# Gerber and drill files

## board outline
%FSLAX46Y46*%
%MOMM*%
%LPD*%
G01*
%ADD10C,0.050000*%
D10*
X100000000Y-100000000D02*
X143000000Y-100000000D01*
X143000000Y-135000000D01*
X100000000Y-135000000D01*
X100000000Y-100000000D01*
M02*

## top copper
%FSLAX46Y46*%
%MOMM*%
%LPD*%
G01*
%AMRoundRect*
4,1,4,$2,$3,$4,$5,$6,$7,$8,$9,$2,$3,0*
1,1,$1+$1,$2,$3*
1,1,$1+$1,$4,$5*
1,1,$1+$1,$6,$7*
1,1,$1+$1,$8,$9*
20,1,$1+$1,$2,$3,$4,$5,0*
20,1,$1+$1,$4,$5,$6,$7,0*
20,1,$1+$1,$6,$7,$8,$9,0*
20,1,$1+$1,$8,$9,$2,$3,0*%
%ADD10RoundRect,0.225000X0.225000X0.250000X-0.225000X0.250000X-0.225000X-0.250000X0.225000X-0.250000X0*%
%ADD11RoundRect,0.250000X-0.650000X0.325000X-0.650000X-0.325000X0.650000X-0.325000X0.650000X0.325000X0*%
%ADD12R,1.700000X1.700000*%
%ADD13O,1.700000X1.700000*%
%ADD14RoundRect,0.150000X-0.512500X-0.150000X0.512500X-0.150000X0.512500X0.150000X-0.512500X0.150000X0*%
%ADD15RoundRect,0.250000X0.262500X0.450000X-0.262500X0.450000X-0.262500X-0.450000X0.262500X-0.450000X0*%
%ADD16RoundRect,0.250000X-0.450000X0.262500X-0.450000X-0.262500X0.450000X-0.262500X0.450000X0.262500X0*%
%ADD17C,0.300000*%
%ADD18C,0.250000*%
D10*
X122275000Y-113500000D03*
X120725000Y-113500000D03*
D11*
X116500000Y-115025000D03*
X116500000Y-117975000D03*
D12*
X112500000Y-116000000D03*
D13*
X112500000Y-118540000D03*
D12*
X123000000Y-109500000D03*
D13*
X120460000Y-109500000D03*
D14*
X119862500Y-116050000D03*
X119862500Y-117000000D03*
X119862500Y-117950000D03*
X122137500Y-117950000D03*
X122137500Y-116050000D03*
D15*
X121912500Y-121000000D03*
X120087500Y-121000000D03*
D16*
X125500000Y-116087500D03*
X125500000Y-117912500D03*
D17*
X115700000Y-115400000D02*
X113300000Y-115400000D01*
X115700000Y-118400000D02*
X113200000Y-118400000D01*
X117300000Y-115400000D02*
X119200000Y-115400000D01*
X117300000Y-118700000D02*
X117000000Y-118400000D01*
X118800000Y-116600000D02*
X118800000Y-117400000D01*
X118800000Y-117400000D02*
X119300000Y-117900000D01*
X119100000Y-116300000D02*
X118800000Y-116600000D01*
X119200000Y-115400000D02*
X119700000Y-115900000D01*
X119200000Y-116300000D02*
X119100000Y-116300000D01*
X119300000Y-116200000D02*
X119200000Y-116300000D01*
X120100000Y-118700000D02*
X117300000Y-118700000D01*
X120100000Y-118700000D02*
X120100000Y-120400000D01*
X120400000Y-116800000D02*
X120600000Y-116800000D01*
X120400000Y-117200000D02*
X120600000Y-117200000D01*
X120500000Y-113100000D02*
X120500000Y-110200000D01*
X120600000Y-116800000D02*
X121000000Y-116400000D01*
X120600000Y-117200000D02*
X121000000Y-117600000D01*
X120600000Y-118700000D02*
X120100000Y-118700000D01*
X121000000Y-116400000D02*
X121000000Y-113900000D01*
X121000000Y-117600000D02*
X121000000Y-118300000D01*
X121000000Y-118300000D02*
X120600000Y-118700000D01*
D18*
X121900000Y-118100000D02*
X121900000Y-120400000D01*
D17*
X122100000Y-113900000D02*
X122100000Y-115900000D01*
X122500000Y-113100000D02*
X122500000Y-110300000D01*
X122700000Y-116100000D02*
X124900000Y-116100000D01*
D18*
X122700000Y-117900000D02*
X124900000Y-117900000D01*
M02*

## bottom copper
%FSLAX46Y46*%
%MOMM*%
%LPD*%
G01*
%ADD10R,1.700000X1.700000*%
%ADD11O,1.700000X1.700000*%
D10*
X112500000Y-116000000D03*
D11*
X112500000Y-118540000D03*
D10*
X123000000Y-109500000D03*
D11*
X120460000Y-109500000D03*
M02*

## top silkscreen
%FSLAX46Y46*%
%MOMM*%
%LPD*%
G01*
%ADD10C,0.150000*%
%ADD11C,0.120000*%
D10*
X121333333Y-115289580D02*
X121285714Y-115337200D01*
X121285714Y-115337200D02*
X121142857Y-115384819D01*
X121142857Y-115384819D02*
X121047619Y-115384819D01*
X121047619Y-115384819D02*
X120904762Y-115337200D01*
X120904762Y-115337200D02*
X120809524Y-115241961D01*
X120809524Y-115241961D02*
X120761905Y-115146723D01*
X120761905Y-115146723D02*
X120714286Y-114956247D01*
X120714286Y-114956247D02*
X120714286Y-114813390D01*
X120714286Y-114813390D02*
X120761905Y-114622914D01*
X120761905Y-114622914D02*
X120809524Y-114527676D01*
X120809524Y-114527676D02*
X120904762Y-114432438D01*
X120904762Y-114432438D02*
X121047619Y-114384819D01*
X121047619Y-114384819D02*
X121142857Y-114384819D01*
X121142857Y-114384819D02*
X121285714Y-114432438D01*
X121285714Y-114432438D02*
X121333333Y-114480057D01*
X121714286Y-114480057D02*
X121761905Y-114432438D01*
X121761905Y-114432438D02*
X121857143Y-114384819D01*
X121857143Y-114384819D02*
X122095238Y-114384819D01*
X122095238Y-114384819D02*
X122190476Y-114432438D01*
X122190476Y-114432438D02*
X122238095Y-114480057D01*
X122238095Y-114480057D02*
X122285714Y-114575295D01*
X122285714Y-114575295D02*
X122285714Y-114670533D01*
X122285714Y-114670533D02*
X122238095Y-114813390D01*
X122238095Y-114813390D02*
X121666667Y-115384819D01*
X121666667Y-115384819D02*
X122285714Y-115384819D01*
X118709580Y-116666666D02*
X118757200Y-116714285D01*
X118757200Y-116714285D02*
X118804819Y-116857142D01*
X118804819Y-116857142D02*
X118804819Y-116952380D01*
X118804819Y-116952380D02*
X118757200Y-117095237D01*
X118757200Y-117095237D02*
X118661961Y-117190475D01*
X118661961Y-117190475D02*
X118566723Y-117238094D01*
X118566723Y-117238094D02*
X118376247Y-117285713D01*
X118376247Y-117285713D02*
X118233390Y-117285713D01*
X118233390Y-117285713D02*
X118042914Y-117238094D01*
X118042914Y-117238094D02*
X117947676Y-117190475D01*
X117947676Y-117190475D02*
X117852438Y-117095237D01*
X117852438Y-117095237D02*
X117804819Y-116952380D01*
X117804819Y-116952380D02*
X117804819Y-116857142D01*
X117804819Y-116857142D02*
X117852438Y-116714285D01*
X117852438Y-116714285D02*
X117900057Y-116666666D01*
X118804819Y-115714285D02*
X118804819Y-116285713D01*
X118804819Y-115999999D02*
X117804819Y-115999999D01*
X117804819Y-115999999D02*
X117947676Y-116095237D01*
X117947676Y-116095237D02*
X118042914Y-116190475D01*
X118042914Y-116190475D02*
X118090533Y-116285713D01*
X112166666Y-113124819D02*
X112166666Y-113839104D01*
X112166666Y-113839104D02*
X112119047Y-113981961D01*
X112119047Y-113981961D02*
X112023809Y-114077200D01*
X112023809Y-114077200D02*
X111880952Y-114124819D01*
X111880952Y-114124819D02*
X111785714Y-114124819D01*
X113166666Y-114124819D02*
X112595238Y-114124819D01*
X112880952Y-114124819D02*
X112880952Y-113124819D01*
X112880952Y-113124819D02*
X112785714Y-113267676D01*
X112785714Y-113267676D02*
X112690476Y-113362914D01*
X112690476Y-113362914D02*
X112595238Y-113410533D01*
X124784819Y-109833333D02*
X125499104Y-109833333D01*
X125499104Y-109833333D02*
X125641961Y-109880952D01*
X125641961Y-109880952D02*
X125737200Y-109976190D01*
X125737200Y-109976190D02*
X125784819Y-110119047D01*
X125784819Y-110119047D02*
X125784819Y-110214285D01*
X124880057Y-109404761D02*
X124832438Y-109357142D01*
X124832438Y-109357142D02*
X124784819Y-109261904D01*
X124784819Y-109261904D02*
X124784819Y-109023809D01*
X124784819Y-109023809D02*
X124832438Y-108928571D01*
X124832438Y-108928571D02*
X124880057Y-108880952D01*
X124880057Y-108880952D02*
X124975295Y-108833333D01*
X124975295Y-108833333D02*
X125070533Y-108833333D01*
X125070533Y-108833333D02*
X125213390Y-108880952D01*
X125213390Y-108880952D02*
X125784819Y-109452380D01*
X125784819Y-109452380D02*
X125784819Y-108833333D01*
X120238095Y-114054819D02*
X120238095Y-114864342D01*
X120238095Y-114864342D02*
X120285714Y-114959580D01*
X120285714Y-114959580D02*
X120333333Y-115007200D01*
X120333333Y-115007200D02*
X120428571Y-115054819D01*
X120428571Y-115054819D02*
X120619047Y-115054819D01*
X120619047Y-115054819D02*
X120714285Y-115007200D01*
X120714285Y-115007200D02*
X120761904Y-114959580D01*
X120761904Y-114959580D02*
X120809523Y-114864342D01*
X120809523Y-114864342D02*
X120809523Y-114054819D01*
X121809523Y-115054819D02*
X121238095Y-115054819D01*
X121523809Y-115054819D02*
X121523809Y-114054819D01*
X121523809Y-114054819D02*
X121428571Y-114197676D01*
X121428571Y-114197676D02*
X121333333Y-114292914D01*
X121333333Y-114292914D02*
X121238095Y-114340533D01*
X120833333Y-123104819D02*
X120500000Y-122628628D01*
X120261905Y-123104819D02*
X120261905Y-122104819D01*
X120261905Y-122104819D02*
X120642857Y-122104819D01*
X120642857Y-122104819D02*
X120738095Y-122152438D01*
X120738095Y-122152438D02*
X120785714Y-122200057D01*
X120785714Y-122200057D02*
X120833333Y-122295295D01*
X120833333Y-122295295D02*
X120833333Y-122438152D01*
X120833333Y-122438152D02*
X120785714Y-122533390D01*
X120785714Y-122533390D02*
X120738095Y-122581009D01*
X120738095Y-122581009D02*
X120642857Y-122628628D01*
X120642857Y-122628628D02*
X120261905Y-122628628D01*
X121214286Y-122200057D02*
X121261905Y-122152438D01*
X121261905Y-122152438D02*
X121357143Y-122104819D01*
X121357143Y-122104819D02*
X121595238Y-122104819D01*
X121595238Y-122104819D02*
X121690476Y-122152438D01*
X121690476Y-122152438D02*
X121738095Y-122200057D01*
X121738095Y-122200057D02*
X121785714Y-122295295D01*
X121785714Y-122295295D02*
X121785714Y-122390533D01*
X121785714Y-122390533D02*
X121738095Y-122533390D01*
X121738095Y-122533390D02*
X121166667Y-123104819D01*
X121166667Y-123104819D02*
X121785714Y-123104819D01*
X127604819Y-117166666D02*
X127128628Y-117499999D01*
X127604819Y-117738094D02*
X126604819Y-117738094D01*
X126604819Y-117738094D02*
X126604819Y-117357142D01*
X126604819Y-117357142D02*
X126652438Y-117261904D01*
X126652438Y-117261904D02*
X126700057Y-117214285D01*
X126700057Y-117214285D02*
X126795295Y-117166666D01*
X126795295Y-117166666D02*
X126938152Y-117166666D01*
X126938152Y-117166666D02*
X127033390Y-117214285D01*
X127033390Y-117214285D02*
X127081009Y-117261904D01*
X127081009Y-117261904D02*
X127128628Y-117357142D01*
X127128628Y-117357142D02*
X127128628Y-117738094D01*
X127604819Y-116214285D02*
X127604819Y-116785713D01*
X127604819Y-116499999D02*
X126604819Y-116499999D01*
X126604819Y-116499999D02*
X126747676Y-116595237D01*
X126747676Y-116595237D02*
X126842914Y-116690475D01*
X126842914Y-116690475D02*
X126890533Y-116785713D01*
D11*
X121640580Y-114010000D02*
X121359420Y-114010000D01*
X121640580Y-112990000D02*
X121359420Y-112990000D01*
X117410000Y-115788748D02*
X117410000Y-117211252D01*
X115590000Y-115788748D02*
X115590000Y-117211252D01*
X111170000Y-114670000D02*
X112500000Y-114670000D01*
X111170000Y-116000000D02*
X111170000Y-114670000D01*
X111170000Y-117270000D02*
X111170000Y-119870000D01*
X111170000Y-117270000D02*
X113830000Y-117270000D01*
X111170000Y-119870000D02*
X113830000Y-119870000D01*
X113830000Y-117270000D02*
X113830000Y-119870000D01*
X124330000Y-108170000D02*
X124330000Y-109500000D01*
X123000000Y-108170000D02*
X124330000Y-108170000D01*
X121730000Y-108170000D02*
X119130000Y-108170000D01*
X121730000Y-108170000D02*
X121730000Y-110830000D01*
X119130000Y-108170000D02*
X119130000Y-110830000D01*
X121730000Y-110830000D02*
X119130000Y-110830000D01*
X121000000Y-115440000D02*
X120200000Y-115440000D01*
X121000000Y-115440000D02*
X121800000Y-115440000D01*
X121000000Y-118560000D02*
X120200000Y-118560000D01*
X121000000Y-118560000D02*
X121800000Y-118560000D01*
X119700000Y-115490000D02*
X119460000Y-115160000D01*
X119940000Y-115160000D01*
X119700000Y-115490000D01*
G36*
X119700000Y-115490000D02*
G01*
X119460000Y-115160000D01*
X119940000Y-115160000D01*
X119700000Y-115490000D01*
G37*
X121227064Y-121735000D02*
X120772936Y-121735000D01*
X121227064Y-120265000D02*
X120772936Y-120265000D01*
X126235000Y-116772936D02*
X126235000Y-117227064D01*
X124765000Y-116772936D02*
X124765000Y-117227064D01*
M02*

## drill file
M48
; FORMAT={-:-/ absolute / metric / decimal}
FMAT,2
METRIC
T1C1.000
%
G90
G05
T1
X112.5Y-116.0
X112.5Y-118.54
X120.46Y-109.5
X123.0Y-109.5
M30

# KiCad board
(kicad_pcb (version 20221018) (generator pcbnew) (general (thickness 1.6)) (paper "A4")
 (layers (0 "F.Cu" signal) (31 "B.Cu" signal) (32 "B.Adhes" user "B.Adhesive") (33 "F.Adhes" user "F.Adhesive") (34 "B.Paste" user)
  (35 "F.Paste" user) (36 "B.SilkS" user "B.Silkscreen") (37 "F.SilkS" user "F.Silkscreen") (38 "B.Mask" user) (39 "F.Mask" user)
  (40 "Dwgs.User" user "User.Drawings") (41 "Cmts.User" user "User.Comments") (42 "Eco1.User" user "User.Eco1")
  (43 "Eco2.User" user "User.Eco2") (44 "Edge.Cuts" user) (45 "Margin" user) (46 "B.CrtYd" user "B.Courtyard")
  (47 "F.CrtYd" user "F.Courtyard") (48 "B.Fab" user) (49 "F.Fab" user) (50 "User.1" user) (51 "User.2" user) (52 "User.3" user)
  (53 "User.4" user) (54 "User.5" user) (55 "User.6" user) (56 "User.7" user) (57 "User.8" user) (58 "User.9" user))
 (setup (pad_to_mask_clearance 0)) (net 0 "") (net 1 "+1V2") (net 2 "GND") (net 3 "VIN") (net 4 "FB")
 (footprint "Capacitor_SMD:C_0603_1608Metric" (layer "F.Cu") (at 121.5 113.5 180)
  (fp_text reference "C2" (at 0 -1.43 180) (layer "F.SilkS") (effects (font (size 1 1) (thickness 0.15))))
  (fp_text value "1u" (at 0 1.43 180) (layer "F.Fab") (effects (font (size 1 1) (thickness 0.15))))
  (fp_line (start -0.14058 -0.51) (end 0.14058 -0.51) (stroke (width 0.12) (type solid)) (layer "F.SilkS"))
  (fp_line (start -0.14058 0.51) (end 0.14058 0.51) (stroke (width 0.12) (type solid)) (layer "F.SilkS"))
  (pad "1" smd roundrect (at -0.775 0 180) (size 0.9 0.95) (layers "F.Cu" "F.Paste" "F.Mask") (roundrect_rratio 0.25) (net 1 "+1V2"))
  (pad "2" smd roundrect (at 0.775 0 180) (size 0.9 0.95) (layers "F.Cu" "F.Paste" "F.Mask") (roundrect_rratio 0.25) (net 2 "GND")))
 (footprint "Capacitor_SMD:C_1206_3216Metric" (layer "F.Cu") (at 116.5 116.5 -90)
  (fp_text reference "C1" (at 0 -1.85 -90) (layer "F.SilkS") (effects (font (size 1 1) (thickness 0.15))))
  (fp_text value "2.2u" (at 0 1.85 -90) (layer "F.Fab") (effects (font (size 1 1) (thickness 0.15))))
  (fp_line (start -0.711252 -0.91) (end 0.711252 -0.91) (stroke (width 0.12) (type solid)) (layer "F.SilkS"))
  (fp_line (start -0.711252 0.91) (end 0.711252 0.91) (stroke (width 0.12) (type solid)) (layer "F.SilkS"))
  (pad "1" smd roundrect (at -1.475 0 270) (size 1.15 1.8) (layers "F.Cu" "F.Paste" "F.Mask") (roundrect_rratio 0.217391) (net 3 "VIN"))
  (pad "2" smd roundrect (at 1.475 0 270) (size 1.15 1.8) (layers "F.Cu" "F.Paste" "F.Mask") (roundrect_rratio 0.217391) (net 2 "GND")))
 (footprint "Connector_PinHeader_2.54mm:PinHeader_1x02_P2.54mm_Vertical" (layer "F.Cu") (at 112.5 116)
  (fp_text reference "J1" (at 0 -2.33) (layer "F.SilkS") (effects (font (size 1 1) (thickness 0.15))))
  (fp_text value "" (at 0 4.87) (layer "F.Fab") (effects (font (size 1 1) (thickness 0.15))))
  (fp_line (start -1.33 -1.33) (end 0 -1.33) (stroke (width 0.12) (type solid)) (layer "F.SilkS"))
  (fp_line (start -1.33 0) (end -1.33 -1.33) (stroke (width 0.12) (type solid)) (layer "F.SilkS"))
  (fp_line (start -1.33 1.27) (end -1.33 3.87) (stroke (width 0.12) (type solid)) (layer "F.SilkS"))
  (fp_line (start -1.33 1.27) (end 1.33 1.27) (stroke (width 0.12) (type solid)) (layer "F.SilkS"))
  (fp_line (start -1.33 3.87) (end 1.33 3.87) (stroke (width 0.12) (type solid)) (layer "F.SilkS"))
  (fp_line (start 1.33 1.27) (end 1.33 3.87) (stroke (width 0.12) (type solid)) (layer "F.SilkS"))
  (pad "1" thru_hole rect (at 0 0) (size 1.7 1.7) (drill 1) (layers "*.Cu" "*.Mask") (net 3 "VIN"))
  (pad "2" thru_hole oval (at 0 2.54) (size 1.7 1.7) (drill 1) (layers "*.Cu" "*.Mask") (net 2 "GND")))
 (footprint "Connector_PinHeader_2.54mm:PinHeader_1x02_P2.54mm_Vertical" (layer "F.Cu") (at 123 109.5 -90)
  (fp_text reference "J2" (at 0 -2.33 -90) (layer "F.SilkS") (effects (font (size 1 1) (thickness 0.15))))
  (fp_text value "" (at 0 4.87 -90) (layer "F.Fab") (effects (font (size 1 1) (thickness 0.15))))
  (fp_line (start -1.33 -1.33) (end 0 -1.33) (stroke (width 0.12) (type solid)) (layer "F.SilkS"))
  (fp_line (start -1.33 0) (end -1.33 -1.33) (stroke (width 0.12) (type solid)) (layer "F.SilkS"))
  (fp_line (start -1.33 1.27) (end -1.33 3.87) (stroke (width 0.12) (type solid)) (layer "F.SilkS"))
  (fp_line (start -1.33 1.27) (end 1.33 1.27) (stroke (width 0.12) (type solid)) (layer "F.SilkS"))
  (fp_line (start -1.33 3.87) (end 1.33 3.87) (stroke (width 0.12) (type solid)) (layer "F.SilkS"))
  (fp_line (start 1.33 1.27) (end 1.33 3.87) (stroke (width 0.12) (type solid)) (layer "F.SilkS"))
  (pad "1" thru_hole rect (at 0 0 270) (size 1.7 1.7) (drill 1) (layers "*.Cu" "*.Mask") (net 1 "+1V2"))
  (pad "2" thru_hole oval (at 0 2.54 270) (size 1.7 1.7) (drill 1) (layers "*.Cu" "*.Mask") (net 2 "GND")))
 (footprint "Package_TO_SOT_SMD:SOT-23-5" (layer "F.Cu") (at 121 117)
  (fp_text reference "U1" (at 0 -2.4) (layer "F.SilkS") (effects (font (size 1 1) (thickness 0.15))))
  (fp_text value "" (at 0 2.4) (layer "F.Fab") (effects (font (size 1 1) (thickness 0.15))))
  (fp_line (start 0 -1.56) (end -0.8 -1.56) (stroke (width 0.12) (type solid)) (layer "F.SilkS"))
  (fp_line (start 0 -1.56) (end 0.8 -1.56) (stroke (width 0.12) (type solid)) (layer "F.SilkS"))
  (fp_line (start 0 1.56) (end -0.8 1.56) (stroke (width 0.12) (type solid)) (layer "F.SilkS"))
  (fp_line (start 0 1.56) (end 0.8 1.56) (stroke (width 0.12) (type solid)) (layer "F.SilkS"))
  (fp_poly
   (pts (xy -1.3 -1.51) (xy -1.54 -1.84) (xy -1.06 -1.84) (xy -1.3 -1.51)) (stroke (width 0.12) (type solid)) (fill solid) (layer "F.SilkS"))
  (pad "1" smd roundrect (at -1.1375 -0.95) (size 1.325 0.6) (layers "F.Cu" "F.Paste" "F.Mask") (roundrect_rratio 0.25) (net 3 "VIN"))
  (pad "2" smd roundrect (at -1.1375 0) (size 1.325 0.6) (layers "F.Cu" "F.Paste" "F.Mask") (roundrect_rratio 0.25) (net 2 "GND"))
  (pad "3" smd roundrect (at -1.1375 0.95) (size 1.325 0.6) (layers "F.Cu" "F.Paste" "F.Mask") (roundrect_rratio 0.25) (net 3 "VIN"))
  (pad "4" smd roundrect (at 1.1375 0.95) (size 1.325 0.6) (layers "F.Cu" "F.Paste" "F.Mask") (roundrect_rratio 0.25) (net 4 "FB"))
  (pad "5" smd roundrect (at 1.1375 -0.95) (size 1.325 0.6) (layers "F.Cu" "F.Paste" "F.Mask") (roundrect_rratio 0.25) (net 1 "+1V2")))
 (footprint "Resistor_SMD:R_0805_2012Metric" (layer "F.Cu") (at 121 121 180)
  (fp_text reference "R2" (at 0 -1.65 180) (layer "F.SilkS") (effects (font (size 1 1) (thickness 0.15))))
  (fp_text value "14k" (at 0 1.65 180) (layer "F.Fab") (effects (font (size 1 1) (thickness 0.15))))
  (fp_line (start -0.227064 -0.735) (end 0.227064 -0.735) (stroke (width 0.12) (type solid)) (layer "F.SilkS"))
  (fp_line (start -0.227064 0.735) (end 0.227064 0.735) (stroke (width 0.12) (type solid)) (layer "F.SilkS"))
  (pad "1" smd roundrect (at -0.9125 0 180) (size 1.025 1.4) (layers "F.Cu" "F.Paste" "F.Mask") (roundrect_rratio 0.243902) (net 4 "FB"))
  (pad "2" smd roundrect (at 0.9125 0 180) (size 1.025 1.4) (layers "F.Cu" "F.Paste" "F.Mask") (roundrect_rratio 0.243902) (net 2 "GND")))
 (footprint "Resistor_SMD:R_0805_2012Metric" (layer "F.Cu") (at 125.5 117 -90)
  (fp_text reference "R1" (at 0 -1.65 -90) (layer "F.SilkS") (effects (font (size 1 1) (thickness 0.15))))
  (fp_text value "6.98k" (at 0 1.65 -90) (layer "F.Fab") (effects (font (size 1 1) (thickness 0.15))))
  (fp_line (start -0.227064 -0.735) (end 0.227064 -0.735) (stroke (width 0.12) (type solid)) (layer "F.SilkS"))
  (fp_line (start -0.227064 0.735) (end 0.227064 0.735) (stroke (width 0.12) (type solid)) (layer "F.SilkS"))
  (pad "1" smd roundrect (at -0.9125 0 270) (size 1.025 1.4) (layers "F.Cu" "F.Paste" "F.Mask") (roundrect_rratio 0.243902) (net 1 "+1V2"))
  (pad "2" smd roundrect (at 0.9125 0 270) (size 1.025 1.4) (layers "F.Cu" "F.Paste" "F.Mask") (roundrect_rratio 0.243902) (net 4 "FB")))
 (gr_rect (start 100 100) (end 143 135) (stroke (width 0.05) (type default)) (fill none) (layer "Edge.Cuts"))
 (segment (start 115.7 115.4) (end 113.3 115.4) (width 0.3) (layer "F.Cu") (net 3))
 (segment (start 115.7 118.4) (end 113.2 118.4) (width 0.3) (layer "F.Cu") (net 2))
 (segment (start 117.3 115.4) (end 119.2 115.4) (width 0.3) (layer "F.Cu") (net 3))
 (segment (start 117.3 118.7) (end 117 118.4) (width 0.3) (layer "F.Cu") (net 2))
 (segment (start 118.8 116.6) (end 118.8 117.4) (width 0.3) (layer "F.Cu") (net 3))
 (segment (start 118.8 117.4) (end 119.3 117.9) (width 0.3) (layer "F.Cu") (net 3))
 (segment (start 119.1 116.3) (end 118.8 116.6) (width 0.3) (layer "F.Cu") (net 3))
 (segment (start 119.2 115.4) (end 119.7 115.9) (width 0.3) (layer "F.Cu") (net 3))
 (segment (start 119.2 116.3) (end 119.1 116.3) (width 0.3) (layer "F.Cu") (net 3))
 (segment (start 119.3 116.2) (end 119.2 116.3) (width 0.3) (layer "F.Cu") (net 3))
 (segment (start 120.1 118.7) (end 117.3 118.7) (width 0.3) (layer "F.Cu") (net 2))
 (segment (start 120.1 118.7) (end 120.1 120.4) (width 0.3) (layer "F.Cu") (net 2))
 (segment (start 120.4 116.8) (end 120.6 116.8) (width 0.3) (layer "F.Cu") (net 2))
 (segment (start 120.4 117.2) (end 120.6 117.2) (width 0.3) (layer "F.Cu") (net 2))
 (segment (start 120.5 113.1) (end 120.5 110.2) (width 0.3) (layer "F.Cu") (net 2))
 (segment (start 120.6 116.8) (end 121 116.4) (width 0.3) (layer "F.Cu") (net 2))
 (segment (start 120.6 117.2) (end 121 117.6) (width 0.3) (layer "F.Cu") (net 2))
 (segment (start 120.6 118.7) (end 120.1 118.7) (width 0.3) (layer "F.Cu") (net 2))
 (segment (start 121 116.4) (end 121 113.9) (width 0.3) (layer "F.Cu") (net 2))
 (segment (start 121 117.6) (end 121 118.3) (width 0.3) (layer "F.Cu") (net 2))
 (segment (start 121 118.3) (end 120.6 118.7) (width 0.3) (layer "F.Cu") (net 2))
 (segment (start 121.9 118.1) (end 121.9 120.4) (width 0.25) (layer "F.Cu") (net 4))
 (segment (start 122.1 113.9) (end 122.1 115.9) (width 0.3) (layer "F.Cu") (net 1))
 (segment (start 122.5 113.1) (end 122.5 110.3) (width 0.3) (layer "F.Cu") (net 1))
 (segment (start 122.7 116.1) (end 124.9 116.1) (width 0.3) (layer "F.Cu") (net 1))
 (segment (start 122.7 117.9) (end 124.9 117.9) (width 0.25) (layer "F.Cu") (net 4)))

